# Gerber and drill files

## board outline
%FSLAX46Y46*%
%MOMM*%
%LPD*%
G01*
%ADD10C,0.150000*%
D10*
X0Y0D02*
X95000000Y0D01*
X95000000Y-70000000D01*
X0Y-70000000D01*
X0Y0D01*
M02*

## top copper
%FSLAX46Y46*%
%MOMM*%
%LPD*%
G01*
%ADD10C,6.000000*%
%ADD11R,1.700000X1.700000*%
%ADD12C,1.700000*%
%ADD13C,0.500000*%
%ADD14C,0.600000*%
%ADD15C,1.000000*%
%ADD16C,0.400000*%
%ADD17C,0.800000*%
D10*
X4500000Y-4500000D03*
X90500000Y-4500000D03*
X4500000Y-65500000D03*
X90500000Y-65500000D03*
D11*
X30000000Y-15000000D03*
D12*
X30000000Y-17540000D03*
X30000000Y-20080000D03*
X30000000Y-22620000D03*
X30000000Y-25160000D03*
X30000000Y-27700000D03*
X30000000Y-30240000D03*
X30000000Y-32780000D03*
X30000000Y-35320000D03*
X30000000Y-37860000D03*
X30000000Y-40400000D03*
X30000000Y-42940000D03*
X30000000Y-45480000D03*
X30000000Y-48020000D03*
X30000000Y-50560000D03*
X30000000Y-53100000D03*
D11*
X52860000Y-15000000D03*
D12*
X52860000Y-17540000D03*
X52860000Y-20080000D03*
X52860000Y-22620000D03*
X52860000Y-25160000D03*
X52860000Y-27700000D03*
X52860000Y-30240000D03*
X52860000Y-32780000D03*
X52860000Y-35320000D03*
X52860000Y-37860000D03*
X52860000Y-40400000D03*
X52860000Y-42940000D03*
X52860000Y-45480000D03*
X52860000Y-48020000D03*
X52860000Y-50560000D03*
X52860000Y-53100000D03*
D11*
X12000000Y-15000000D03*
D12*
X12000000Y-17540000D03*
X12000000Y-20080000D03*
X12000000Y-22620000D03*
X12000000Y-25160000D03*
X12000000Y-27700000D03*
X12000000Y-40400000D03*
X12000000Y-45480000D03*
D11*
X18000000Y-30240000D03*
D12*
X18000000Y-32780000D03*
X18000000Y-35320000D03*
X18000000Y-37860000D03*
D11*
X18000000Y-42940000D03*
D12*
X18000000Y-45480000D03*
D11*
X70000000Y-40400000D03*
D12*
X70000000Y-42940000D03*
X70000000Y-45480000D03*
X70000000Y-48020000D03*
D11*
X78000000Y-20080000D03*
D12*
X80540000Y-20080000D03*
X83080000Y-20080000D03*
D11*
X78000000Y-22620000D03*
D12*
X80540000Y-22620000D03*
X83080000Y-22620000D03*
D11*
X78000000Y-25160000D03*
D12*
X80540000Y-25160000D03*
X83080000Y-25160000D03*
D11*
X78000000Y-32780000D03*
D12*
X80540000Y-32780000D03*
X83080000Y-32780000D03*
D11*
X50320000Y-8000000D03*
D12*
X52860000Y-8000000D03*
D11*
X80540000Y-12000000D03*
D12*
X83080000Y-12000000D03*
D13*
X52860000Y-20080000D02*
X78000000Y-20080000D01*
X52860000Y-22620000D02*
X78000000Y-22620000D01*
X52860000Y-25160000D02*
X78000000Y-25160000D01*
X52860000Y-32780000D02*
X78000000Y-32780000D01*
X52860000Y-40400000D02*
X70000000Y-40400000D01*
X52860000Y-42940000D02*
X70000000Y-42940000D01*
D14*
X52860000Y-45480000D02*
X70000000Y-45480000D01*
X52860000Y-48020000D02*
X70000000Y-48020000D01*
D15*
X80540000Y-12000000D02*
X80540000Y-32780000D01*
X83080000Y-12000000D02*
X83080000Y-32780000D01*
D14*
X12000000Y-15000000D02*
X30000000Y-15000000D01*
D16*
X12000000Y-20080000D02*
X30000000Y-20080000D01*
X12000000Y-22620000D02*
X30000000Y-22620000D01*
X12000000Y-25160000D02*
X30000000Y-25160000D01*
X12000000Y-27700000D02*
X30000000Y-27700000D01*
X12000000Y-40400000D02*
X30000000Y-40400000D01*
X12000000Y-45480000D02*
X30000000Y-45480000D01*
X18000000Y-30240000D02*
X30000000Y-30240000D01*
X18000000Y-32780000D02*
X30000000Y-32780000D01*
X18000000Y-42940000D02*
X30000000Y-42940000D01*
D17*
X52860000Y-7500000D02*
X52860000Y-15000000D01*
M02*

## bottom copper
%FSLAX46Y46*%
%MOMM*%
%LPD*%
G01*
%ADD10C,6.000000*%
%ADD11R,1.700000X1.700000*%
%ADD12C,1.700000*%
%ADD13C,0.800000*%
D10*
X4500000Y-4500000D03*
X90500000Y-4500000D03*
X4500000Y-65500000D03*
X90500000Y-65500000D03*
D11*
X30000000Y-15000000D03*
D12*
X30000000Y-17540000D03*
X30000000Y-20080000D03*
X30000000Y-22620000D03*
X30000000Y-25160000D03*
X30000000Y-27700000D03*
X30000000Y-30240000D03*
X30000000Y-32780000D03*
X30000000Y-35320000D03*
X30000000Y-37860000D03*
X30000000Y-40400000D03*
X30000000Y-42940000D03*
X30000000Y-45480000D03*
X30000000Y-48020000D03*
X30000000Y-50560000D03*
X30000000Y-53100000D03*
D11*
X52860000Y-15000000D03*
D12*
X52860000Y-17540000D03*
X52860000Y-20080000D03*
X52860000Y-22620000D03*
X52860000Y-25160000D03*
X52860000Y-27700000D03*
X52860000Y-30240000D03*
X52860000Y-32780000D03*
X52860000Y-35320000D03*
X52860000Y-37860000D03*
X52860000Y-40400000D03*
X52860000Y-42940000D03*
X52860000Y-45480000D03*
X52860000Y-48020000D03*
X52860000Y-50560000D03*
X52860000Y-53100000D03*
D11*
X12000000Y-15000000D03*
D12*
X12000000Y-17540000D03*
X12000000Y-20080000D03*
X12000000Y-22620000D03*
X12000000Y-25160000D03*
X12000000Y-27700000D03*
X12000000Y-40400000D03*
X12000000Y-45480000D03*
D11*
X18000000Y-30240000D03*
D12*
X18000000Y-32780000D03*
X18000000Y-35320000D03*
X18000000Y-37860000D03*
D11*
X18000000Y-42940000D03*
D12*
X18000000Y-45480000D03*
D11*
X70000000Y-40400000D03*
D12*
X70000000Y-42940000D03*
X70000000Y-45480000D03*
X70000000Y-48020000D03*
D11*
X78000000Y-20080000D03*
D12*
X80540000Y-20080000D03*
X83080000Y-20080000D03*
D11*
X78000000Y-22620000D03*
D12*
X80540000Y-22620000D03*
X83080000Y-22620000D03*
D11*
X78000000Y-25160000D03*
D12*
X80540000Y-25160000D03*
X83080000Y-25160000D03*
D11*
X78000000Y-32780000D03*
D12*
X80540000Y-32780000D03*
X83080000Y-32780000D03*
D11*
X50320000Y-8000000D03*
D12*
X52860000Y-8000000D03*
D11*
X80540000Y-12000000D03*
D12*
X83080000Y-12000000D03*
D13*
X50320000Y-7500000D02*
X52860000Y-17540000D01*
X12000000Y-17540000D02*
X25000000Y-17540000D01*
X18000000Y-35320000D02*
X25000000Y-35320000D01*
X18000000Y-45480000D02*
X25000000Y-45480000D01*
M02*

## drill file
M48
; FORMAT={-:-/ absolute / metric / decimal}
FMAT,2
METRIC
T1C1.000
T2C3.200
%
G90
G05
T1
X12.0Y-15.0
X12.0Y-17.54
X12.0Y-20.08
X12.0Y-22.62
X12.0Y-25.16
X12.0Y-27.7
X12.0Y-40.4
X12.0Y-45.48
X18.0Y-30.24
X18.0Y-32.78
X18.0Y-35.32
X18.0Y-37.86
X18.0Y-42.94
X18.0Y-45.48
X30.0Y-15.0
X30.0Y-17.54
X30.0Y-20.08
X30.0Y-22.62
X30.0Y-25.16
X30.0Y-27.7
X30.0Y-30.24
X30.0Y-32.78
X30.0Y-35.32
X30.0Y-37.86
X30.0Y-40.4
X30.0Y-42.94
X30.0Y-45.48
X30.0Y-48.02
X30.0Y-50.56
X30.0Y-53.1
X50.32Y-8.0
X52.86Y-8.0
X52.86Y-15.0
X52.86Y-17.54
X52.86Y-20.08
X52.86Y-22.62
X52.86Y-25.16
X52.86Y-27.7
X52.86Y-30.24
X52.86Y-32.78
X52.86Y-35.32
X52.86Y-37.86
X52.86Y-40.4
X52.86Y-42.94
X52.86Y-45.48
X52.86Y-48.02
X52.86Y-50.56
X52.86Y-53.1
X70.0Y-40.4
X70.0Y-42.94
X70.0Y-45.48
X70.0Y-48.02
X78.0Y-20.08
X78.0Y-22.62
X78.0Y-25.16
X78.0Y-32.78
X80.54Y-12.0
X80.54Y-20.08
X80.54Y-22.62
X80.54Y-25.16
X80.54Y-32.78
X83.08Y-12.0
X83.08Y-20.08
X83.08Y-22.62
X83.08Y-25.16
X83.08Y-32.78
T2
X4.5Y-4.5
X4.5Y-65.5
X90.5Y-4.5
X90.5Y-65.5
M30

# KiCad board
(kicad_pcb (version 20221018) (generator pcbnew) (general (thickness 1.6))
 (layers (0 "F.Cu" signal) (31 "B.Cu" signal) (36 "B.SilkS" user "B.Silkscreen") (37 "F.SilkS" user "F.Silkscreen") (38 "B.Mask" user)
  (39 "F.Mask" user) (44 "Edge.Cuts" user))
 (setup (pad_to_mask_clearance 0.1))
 (gr_rect (start 0 0) (end 95.0 70.0) (layer "Edge.Cuts") (width 0.15) (fill none))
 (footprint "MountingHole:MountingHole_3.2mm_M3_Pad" (layer "F.Cu") (at 4.5 4.5)
  (pad "" np_thru_hole circle (at 0 0) (size 6.0 6.0) (drill 3.2) (layers *.Cu *.Mask)))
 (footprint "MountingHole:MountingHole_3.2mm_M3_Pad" (layer "F.Cu") (at 90.5 4.5)
  (pad "" np_thru_hole circle (at 0 0) (size 6.0 6.0) (drill 3.2) (layers *.Cu *.Mask)))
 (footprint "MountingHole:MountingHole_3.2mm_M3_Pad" (layer "F.Cu") (at 4.5 65.5)
  (pad "" np_thru_hole circle (at 0 0) (size 6.0 6.0) (drill 3.2) (layers *.Cu *.Mask)))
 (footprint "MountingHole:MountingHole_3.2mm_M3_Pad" (layer "F.Cu") (at 90.5 65.5)
  (pad "" np_thru_hole circle (at 0 0) (size 6.0 6.0) (drill 3.2) (layers *.Cu *.Mask)))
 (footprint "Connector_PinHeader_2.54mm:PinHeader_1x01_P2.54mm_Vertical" (layer "F.Cu") (at 30.0 15.0)
  (pad "1" thru_hole rect (at 0 0) (size 1.7 1.7) (drill 1.0) (layers *.Cu *.Mask "F.SilkS")))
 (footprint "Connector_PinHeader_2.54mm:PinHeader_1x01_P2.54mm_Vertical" (layer "F.Cu") (at 30.0 17.54)
  (pad "1" thru_hole circle (at 0 0) (size 1.7 1.7) (drill 1.0) (layers *.Cu *.Mask "F.SilkS")))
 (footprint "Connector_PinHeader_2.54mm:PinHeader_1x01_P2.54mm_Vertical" (layer "F.Cu") (at 30.0 20.08)
  (pad "1" thru_hole circle (at 0 0) (size 1.7 1.7) (drill 1.0) (layers *.Cu *.Mask "F.SilkS")))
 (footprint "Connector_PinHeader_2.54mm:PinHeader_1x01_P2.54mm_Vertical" (layer "F.Cu") (at 30.0 22.62)
  (pad "1" thru_hole circle (at 0 0) (size 1.7 1.7) (drill 1.0) (layers *.Cu *.Mask "F.SilkS")))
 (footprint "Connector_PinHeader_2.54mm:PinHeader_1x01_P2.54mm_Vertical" (layer "F.Cu") (at 30.0 25.16)
  (pad "1" thru_hole circle (at 0 0) (size 1.7 1.7) (drill 1.0) (layers *.Cu *.Mask "F.SilkS")))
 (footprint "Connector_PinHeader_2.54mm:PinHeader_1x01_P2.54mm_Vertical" (layer "F.Cu") (at 30.0 27.7)
  (pad "1" thru_hole circle (at 0 0) (size 1.7 1.7) (drill 1.0) (layers *.Cu *.Mask "F.SilkS")))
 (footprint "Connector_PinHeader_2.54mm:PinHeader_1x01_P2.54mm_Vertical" (layer "F.Cu") (at 30.0 30.240000000000002)
  (pad "1" thru_hole circle (at 0 0) (size 1.7 1.7) (drill 1.0) (layers *.Cu *.Mask "F.SilkS")))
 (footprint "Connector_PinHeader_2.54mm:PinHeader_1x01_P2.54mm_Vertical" (layer "F.Cu") (at 30.0 32.78)
  (pad "1" thru_hole circle (at 0 0) (size 1.7 1.7) (drill 1.0) (layers *.Cu *.Mask "F.SilkS")))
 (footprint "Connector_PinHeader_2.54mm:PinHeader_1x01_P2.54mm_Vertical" (layer "F.Cu") (at 30.0 35.32)
  (pad "1" thru_hole circle (at 0 0) (size 1.7 1.7) (drill 1.0) (layers *.Cu *.Mask "F.SilkS")))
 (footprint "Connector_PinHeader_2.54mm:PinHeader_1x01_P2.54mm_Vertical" (layer "F.Cu") (at 30.0 37.86)
  (pad "1" thru_hole circle (at 0 0) (size 1.7 1.7) (drill 1.0) (layers *.Cu *.Mask "F.SilkS")))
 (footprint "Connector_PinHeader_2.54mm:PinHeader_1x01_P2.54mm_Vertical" (layer "F.Cu") (at 30.0 40.4)
  (pad "1" thru_hole circle (at 0 0) (size 1.7 1.7) (drill 1.0) (layers *.Cu *.Mask "F.SilkS")))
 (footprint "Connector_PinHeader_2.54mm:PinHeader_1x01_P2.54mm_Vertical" (layer "F.Cu") (at 30.0 42.94)
  (pad "1" thru_hole circle (at 0 0) (size 1.7 1.7) (drill 1.0) (layers *.Cu *.Mask "F.SilkS")))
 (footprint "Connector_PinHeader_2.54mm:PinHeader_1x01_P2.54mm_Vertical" (layer "F.Cu") (at 30.0 45.480000000000004)
  (pad "1" thru_hole circle (at 0 0) (size 1.7 1.7) (drill 1.0) (layers *.Cu *.Mask "F.SilkS")))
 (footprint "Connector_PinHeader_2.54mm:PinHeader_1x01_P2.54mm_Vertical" (layer "F.Cu") (at 30.0 48.02)
  (pad "1" thru_hole circle (at 0 0) (size 1.7 1.7) (drill 1.0) (layers *.Cu *.Mask "F.SilkS")))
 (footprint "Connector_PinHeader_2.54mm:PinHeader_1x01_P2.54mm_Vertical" (layer "F.Cu") (at 30.0 50.56)
  (pad "1" thru_hole circle (at 0 0) (size 1.7 1.7) (drill 1.0) (layers *.Cu *.Mask "F.SilkS")))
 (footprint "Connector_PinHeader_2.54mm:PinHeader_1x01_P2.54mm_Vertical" (layer "F.Cu") (at 30.0 53.1)
  (pad "1" thru_hole circle (at 0 0) (size 1.7 1.7) (drill 1.0) (layers *.Cu *.Mask "F.SilkS")))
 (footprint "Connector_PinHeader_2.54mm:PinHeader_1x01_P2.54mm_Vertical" (layer "F.Cu") (at 52.86 15.0)
  (pad "1" thru_hole rect (at 0 0) (size 1.7 1.7) (drill 1.0) (layers *.Cu *.Mask "F.SilkS")))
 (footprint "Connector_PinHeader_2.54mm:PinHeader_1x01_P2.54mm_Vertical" (layer "F.Cu") (at 52.86 17.54)
  (pad "1" thru_hole circle (at 0 0) (size 1.7 1.7) (drill 1.0) (layers *.Cu *.Mask "F.SilkS")))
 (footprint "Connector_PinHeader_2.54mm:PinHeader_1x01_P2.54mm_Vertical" (layer "F.Cu") (at 52.86 20.08)
  (pad "1" thru_hole circle (at 0 0) (size 1.7 1.7) (drill 1.0) (layers *.Cu *.Mask "F.SilkS")))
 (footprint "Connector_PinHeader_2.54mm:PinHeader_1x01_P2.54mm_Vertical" (layer "F.Cu") (at 52.86 22.62)
  (pad "1" thru_hole circle (at 0 0) (size 1.7 1.7) (drill 1.0) (layers *.Cu *.Mask "F.SilkS")))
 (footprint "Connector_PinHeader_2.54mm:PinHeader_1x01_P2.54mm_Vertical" (layer "F.Cu") (at 52.86 25.16)
  (pad "1" thru_hole circle (at 0 0) (size 1.7 1.7) (drill 1.0) (layers *.Cu *.Mask "F.SilkS")))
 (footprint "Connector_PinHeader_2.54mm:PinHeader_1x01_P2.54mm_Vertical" (layer "F.Cu") (at 52.86 27.7)
  (pad "1" thru_hole circle (at 0 0) (size 1.7 1.7) (drill 1.0) (layers *.Cu *.Mask "F.SilkS")))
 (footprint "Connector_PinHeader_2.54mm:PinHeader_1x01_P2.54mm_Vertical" (layer "F.Cu") (at 52.86 30.240000000000002)
  (pad "1" thru_hole circle (at 0 0) (size 1.7 1.7) (drill 1.0) (layers *.Cu *.Mask "F.SilkS")))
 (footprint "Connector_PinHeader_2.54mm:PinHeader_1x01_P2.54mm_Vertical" (layer "F.Cu") (at 52.86 32.78)
  (pad "1" thru_hole circle (at 0 0) (size 1.7 1.7) (drill 1.0) (layers *.Cu *.Mask "F.SilkS")))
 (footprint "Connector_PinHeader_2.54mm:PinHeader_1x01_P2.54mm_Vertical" (layer "F.Cu") (at 52.86 35.32)
  (pad "1" thru_hole circle (at 0 0) (size 1.7 1.7) (drill 1.0) (layers *.Cu *.Mask "F.SilkS")))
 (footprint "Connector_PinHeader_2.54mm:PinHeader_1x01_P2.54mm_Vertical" (layer "F.Cu") (at 52.86 37.86)
  (pad "1" thru_hole circle (at 0 0) (size 1.7 1.7) (drill 1.0) (layers *.Cu *.Mask "F.SilkS")))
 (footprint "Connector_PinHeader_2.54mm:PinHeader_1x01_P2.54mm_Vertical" (layer "F.Cu") (at 52.86 40.4)
  (pad "1" thru_hole circle (at 0 0) (size 1.7 1.7) (drill 1.0) (layers *.Cu *.Mask "F.SilkS")))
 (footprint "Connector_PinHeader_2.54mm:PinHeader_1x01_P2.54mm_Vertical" (layer "F.Cu") (at 52.86 42.94)
  (pad "1" thru_hole circle (at 0 0) (size 1.7 1.7) (drill 1.0) (layers *.Cu *.Mask "F.SilkS")))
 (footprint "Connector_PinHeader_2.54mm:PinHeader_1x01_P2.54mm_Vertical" (layer "F.Cu") (at 52.86 45.480000000000004)
  (pad "1" thru_hole circle (at 0 0) (size 1.7 1.7) (drill 1.0) (layers *.Cu *.Mask "F.SilkS")))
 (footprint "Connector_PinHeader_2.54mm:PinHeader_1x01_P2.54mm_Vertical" (layer "F.Cu") (at 52.86 48.02)
  (pad "1" thru_hole circle (at 0 0) (size 1.7 1.7) (drill 1.0) (layers *.Cu *.Mask "F.SilkS")))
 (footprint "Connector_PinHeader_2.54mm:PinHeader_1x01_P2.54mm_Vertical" (layer "F.Cu") (at 52.86 50.56)
  (pad "1" thru_hole circle (at 0 0) (size 1.7 1.7) (drill 1.0) (layers *.Cu *.Mask "F.SilkS")))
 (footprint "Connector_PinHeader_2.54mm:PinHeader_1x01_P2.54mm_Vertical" (layer "F.Cu") (at 52.86 53.1)
  (pad "1" thru_hole circle (at 0 0) (size 1.7 1.7) (drill 1.0) (layers *.Cu *.Mask "F.SilkS")))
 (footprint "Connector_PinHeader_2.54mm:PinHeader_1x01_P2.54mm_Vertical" (layer "F.Cu") (at 12.0 15.0)
  (pad "1" thru_hole rect (at 0 0) (size 1.7 1.7) (drill 1.0) (layers *.Cu *.Mask "F.SilkS")))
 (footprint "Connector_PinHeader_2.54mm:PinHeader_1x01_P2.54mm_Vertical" (layer "F.Cu") (at 12.0 17.54)
  (pad "1" thru_hole circle (at 0 0) (size 1.7 1.7) (drill 1.0) (layers *.Cu *.Mask "F.SilkS")))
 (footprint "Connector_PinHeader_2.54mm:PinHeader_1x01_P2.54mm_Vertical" (layer "F.Cu") (at 12.0 20.08)
  (pad "1" thru_hole circle (at 0 0) (size 1.7 1.7) (drill 1.0) (layers *.Cu *.Mask "F.SilkS")))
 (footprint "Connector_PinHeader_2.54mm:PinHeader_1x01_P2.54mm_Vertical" (layer "F.Cu") (at 12.0 22.62)
  (pad "1" thru_hole circle (at 0 0) (size 1.7 1.7) (drill 1.0) (layers *.Cu *.Mask "F.SilkS")))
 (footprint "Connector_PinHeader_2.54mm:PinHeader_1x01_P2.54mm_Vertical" (layer "F.Cu") (at 12.0 25.16)
  (pad "1" thru_hole circle (at 0 0) (size 1.7 1.7) (drill 1.0) (layers *.Cu *.Mask "F.SilkS")))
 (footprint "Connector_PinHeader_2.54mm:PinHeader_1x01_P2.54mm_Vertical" (layer "F.Cu") (at 12.0 27.7)
  (pad "1" thru_hole circle (at 0 0) (size 1.7 1.7) (drill 1.0) (layers *.Cu *.Mask "F.SilkS")))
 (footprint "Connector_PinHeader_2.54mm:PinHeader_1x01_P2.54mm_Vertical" (layer "F.Cu") (at 12.0 40.4)
  (pad "1" thru_hole circle (at 0 0) (size 1.7 1.7) (drill 1.0) (layers *.Cu *.Mask "F.SilkS")))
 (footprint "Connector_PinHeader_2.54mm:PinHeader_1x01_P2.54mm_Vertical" (layer "F.Cu") (at 12.0 45.48)
  (pad "1" thru_hole circle (at 0 0) (size 1.7 1.7) (drill 1.0) (layers *.Cu *.Mask "F.SilkS")))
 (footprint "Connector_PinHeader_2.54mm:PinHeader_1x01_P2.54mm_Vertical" (layer "F.Cu") (at 18.0 30.24)
  (pad "1" thru_hole rect (at 0 0) (size 1.7 1.7) (drill 1.0) (layers *.Cu *.Mask "F.SilkS")))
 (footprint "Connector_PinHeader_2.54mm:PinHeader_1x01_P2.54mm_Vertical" (layer "F.Cu") (at 18.0 32.78)
  (pad "1" thru_hole circle (at 0 0) (size 1.7 1.7) (drill 1.0) (layers *.Cu *.Mask "F.SilkS")))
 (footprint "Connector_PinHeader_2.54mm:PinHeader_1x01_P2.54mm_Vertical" (layer "F.Cu") (at 18.0 35.32)
  (pad "1" thru_hole circle (at 0 0) (size 1.7 1.7) (drill 1.0) (layers *.Cu *.Mask "F.SilkS")))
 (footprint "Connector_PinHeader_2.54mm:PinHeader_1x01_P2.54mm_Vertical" (layer "F.Cu") (at 18.0 37.86)
  (pad "1" thru_hole circle (at 0 0) (size 1.7 1.7) (drill 1.0) (layers *.Cu *.Mask "F.SilkS")))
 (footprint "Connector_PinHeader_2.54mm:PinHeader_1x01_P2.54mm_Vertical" (layer "F.Cu") (at 18.0 42.94)
  (pad "1" thru_hole rect (at 0 0) (size 1.7 1.7) (drill 1.0) (layers *.Cu *.Mask "F.SilkS")))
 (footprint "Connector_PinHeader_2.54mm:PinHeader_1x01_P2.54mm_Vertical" (layer "F.Cu") (at 18.0 45.48)
  (pad "1" thru_hole circle (at 0 0) (size 1.7 1.7) (drill 1.0) (layers *.Cu *.Mask "F.SilkS")))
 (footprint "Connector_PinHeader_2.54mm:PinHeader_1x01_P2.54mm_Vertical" (layer "F.Cu") (at 70.0 40.4)
  (pad "1" thru_hole rect (at 0 0) (size 1.7 1.7) (drill 1.0) (layers *.Cu *.Mask "F.SilkS")))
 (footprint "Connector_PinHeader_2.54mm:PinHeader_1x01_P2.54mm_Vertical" (layer "F.Cu") (at 70.0 42.94)
  (pad "1" thru_hole circle (at 0 0) (size 1.7 1.7) (drill 1.0) (layers *.Cu *.Mask "F.SilkS")))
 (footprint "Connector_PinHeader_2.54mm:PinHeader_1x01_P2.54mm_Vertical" (layer "F.Cu") (at 70.0 45.48)
  (pad "1" thru_hole circle (at 0 0) (size 1.7 1.7) (drill 1.0) (layers *.Cu *.Mask "F.SilkS")))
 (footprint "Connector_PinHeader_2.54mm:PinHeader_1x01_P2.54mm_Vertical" (layer "F.Cu") (at 70.0 48.019999999999996)
  (pad "1" thru_hole circle (at 0 0) (size 1.7 1.7) (drill 1.0) (layers *.Cu *.Mask "F.SilkS")))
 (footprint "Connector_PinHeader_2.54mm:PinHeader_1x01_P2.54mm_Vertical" (layer "F.Cu") (at 78.0 20.08)
  (pad "1" thru_hole rect (at 0 0) (size 1.7 1.7) (drill 1.0) (layers *.Cu *.Mask "F.SilkS")))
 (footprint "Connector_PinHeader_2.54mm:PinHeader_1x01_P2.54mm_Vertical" (layer "F.Cu") (at 80.54 20.08)
  (pad "1" thru_hole circle (at 0 0) (size 1.7 1.7) (drill 1.0) (layers *.Cu *.Mask "F.SilkS")))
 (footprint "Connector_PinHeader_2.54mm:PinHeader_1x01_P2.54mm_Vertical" (layer "F.Cu") (at 83.08 20.08)
  (pad "1" thru_hole circle (at 0 0) (size 1.7 1.7) (drill 1.0) (layers *.Cu *.Mask "F.SilkS")))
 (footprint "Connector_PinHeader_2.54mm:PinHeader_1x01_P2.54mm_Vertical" (layer "F.Cu") (at 78.0 22.62)
  (pad "1" thru_hole rect (at 0 0) (size 1.7 1.7) (drill 1.0) (layers *.Cu *.Mask "F.SilkS")))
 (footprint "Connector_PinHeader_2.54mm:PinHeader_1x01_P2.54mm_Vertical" (layer "F.Cu") (at 80.54 22.62)
  (pad "1" thru_hole circle (at 0 0) (size 1.7 1.7) (drill 1.0) (layers *.Cu *.Mask "F.SilkS")))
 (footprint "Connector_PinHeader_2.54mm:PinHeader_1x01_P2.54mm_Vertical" (layer "F.Cu") (at 83.08 22.62)
  (pad "1" thru_hole circle (at 0 0) (size 1.7 1.7) (drill 1.0) (layers *.Cu *.Mask "F.SilkS")))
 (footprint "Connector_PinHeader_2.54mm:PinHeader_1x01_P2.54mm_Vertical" (layer "F.Cu") (at 78.0 25.16)
  (pad "1" thru_hole rect (at 0 0) (size 1.7 1.7) (drill 1.0) (layers *.Cu *.Mask "F.SilkS")))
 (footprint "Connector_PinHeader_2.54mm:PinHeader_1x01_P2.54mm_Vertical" (layer "F.Cu") (at 80.54 25.16)
  (pad "1" thru_hole circle (at 0 0) (size 1.7 1.7) (drill 1.0) (layers *.Cu *.Mask "F.SilkS")))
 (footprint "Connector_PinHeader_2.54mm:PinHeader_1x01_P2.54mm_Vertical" (layer "F.Cu") (at 83.08 25.16)
  (pad "1" thru_hole circle (at 0 0) (size 1.7 1.7) (drill 1.0) (layers *.Cu *.Mask "F.SilkS")))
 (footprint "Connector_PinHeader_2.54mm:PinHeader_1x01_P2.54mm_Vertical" (layer "F.Cu") (at 78.0 32.78)
  (pad "1" thru_hole rect (at 0 0) (size 1.7 1.7) (drill 1.0) (layers *.Cu *.Mask "F.SilkS")))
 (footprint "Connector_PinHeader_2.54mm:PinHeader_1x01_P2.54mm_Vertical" (layer "F.Cu") (at 80.54 32.78)
  (pad "1" thru_hole circle (at 0 0) (size 1.7 1.7) (drill 1.0) (layers *.Cu *.Mask "F.SilkS")))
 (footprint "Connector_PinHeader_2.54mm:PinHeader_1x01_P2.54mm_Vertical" (layer "F.Cu") (at 83.08 32.78)
  (pad "1" thru_hole circle (at 0 0) (size 1.7 1.7) (drill 1.0) (layers *.Cu *.Mask "F.SilkS")))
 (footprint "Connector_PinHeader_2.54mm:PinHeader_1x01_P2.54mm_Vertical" (layer "F.Cu") (at 50.32 8.0)
  (pad "1" thru_hole rect (at 0 0) (size 1.7 1.7) (drill 1.0) (layers *.Cu *.Mask "F.SilkS")))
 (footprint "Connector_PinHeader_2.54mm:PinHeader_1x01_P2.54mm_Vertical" (layer "F.Cu") (at 52.86 8.0)
  (pad "1" thru_hole circle (at 0 0) (size 1.7 1.7) (drill 1.0) (layers *.Cu *.Mask "F.SilkS")))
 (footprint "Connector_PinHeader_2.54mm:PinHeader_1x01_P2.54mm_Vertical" (layer "F.Cu") (at 80.54 12.0)
  (pad "1" thru_hole rect (at 0 0) (size 1.7 1.7) (drill 1.0) (layers *.Cu *.Mask "F.SilkS")))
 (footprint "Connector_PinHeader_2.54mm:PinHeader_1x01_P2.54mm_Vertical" (layer "F.Cu") (at 83.08000000000001 12.0)
  (pad "1" thru_hole circle (at 0 0) (size 1.7 1.7) (drill 1.0) (layers *.Cu *.Mask "F.SilkS")))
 (segment (start 52.86 20.08) (end 78.0 20.08) (width 0.5) (layer "F.Cu") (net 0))
 (segment (start 52.86 22.62) (end 78.0 22.62) (width 0.5) (layer "F.Cu") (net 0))
 (segment (start 52.86 25.16) (end 78.0 25.16) (width 0.5) (layer "F.Cu") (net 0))
 (segment (start 52.86 32.78) (end 78.0 32.78) (width 0.5) (layer "F.Cu") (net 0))
 (segment (start 52.86 40.4) (end 70.0 40.4) (width 0.5) (layer "F.Cu") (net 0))
 (segment (start 52.86 42.94) (end 70.0 42.94) (width 0.5) (layer "F.Cu") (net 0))
 (segment (start 52.86 45.48) (end 70.0 45.48) (width 0.6) (layer "F.Cu") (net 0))
 (segment (start 52.86 48.02) (end 70.0 48.02) (width 0.6) (layer "F.Cu") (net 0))
 (segment (start 80.54 12.0) (end 80.54 32.78) (width 1.0) (layer "F.Cu") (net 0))
 (segment (start 83.08 12.0) (end 83.08 32.78) (width 1.0) (layer "F.Cu") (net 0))
 (segment (start 12.0 15.0) (end 30.0 15.0) (width 0.6) (layer "F.Cu") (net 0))
 (segment (start 12.0 20.08) (end 30.0 20.08) (width 0.4) (layer "F.Cu") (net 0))
 (segment (start 12.0 22.62) (end 30.0 22.62) (width 0.4) (layer "F.Cu") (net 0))
 (segment (start 12.0 25.16) (end 30.0 25.16) (width 0.4) (layer "F.Cu") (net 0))
 (segment (start 12.0 27.7) (end 30.0 27.7) (width 0.4) (layer "F.Cu") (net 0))
 (segment (start 12.0 40.4) (end 30.0 40.4) (width 0.4) (layer "F.Cu") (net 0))
 (segment (start 12.0 45.48) (end 30.0 45.48) (width 0.4) (layer "F.Cu") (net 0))
 (segment (start 18.0 30.24) (end 30.0 30.24) (width 0.4) (layer "F.Cu") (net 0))
 (segment (start 18.0 32.78) (end 30.0 32.78) (width 0.4) (layer "F.Cu") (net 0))
 (segment (start 18.0 42.94) (end 30.0 42.94) (width 0.4) (layer "F.Cu") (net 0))
 (segment (start 52.86 7.5) (end 52.86 15.0) (width 0.8) (layer "F.Cu") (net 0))
 (segment (start 50.32 7.5) (end 52.86 17.54) (width 0.8) (layer "B.Cu") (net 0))
 (segment (start 12.0 17.54) (end 25.0 17.54) (width 0.8) (layer "B.Cu") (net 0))
 (segment (start 18.0 35.32) (end 25.0 35.32) (width 0.8) (layer "B.Cu") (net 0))
 (segment (start 18.0 45.48) (end 25.0 45.48) (width 0.8) (layer "B.Cu") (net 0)))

